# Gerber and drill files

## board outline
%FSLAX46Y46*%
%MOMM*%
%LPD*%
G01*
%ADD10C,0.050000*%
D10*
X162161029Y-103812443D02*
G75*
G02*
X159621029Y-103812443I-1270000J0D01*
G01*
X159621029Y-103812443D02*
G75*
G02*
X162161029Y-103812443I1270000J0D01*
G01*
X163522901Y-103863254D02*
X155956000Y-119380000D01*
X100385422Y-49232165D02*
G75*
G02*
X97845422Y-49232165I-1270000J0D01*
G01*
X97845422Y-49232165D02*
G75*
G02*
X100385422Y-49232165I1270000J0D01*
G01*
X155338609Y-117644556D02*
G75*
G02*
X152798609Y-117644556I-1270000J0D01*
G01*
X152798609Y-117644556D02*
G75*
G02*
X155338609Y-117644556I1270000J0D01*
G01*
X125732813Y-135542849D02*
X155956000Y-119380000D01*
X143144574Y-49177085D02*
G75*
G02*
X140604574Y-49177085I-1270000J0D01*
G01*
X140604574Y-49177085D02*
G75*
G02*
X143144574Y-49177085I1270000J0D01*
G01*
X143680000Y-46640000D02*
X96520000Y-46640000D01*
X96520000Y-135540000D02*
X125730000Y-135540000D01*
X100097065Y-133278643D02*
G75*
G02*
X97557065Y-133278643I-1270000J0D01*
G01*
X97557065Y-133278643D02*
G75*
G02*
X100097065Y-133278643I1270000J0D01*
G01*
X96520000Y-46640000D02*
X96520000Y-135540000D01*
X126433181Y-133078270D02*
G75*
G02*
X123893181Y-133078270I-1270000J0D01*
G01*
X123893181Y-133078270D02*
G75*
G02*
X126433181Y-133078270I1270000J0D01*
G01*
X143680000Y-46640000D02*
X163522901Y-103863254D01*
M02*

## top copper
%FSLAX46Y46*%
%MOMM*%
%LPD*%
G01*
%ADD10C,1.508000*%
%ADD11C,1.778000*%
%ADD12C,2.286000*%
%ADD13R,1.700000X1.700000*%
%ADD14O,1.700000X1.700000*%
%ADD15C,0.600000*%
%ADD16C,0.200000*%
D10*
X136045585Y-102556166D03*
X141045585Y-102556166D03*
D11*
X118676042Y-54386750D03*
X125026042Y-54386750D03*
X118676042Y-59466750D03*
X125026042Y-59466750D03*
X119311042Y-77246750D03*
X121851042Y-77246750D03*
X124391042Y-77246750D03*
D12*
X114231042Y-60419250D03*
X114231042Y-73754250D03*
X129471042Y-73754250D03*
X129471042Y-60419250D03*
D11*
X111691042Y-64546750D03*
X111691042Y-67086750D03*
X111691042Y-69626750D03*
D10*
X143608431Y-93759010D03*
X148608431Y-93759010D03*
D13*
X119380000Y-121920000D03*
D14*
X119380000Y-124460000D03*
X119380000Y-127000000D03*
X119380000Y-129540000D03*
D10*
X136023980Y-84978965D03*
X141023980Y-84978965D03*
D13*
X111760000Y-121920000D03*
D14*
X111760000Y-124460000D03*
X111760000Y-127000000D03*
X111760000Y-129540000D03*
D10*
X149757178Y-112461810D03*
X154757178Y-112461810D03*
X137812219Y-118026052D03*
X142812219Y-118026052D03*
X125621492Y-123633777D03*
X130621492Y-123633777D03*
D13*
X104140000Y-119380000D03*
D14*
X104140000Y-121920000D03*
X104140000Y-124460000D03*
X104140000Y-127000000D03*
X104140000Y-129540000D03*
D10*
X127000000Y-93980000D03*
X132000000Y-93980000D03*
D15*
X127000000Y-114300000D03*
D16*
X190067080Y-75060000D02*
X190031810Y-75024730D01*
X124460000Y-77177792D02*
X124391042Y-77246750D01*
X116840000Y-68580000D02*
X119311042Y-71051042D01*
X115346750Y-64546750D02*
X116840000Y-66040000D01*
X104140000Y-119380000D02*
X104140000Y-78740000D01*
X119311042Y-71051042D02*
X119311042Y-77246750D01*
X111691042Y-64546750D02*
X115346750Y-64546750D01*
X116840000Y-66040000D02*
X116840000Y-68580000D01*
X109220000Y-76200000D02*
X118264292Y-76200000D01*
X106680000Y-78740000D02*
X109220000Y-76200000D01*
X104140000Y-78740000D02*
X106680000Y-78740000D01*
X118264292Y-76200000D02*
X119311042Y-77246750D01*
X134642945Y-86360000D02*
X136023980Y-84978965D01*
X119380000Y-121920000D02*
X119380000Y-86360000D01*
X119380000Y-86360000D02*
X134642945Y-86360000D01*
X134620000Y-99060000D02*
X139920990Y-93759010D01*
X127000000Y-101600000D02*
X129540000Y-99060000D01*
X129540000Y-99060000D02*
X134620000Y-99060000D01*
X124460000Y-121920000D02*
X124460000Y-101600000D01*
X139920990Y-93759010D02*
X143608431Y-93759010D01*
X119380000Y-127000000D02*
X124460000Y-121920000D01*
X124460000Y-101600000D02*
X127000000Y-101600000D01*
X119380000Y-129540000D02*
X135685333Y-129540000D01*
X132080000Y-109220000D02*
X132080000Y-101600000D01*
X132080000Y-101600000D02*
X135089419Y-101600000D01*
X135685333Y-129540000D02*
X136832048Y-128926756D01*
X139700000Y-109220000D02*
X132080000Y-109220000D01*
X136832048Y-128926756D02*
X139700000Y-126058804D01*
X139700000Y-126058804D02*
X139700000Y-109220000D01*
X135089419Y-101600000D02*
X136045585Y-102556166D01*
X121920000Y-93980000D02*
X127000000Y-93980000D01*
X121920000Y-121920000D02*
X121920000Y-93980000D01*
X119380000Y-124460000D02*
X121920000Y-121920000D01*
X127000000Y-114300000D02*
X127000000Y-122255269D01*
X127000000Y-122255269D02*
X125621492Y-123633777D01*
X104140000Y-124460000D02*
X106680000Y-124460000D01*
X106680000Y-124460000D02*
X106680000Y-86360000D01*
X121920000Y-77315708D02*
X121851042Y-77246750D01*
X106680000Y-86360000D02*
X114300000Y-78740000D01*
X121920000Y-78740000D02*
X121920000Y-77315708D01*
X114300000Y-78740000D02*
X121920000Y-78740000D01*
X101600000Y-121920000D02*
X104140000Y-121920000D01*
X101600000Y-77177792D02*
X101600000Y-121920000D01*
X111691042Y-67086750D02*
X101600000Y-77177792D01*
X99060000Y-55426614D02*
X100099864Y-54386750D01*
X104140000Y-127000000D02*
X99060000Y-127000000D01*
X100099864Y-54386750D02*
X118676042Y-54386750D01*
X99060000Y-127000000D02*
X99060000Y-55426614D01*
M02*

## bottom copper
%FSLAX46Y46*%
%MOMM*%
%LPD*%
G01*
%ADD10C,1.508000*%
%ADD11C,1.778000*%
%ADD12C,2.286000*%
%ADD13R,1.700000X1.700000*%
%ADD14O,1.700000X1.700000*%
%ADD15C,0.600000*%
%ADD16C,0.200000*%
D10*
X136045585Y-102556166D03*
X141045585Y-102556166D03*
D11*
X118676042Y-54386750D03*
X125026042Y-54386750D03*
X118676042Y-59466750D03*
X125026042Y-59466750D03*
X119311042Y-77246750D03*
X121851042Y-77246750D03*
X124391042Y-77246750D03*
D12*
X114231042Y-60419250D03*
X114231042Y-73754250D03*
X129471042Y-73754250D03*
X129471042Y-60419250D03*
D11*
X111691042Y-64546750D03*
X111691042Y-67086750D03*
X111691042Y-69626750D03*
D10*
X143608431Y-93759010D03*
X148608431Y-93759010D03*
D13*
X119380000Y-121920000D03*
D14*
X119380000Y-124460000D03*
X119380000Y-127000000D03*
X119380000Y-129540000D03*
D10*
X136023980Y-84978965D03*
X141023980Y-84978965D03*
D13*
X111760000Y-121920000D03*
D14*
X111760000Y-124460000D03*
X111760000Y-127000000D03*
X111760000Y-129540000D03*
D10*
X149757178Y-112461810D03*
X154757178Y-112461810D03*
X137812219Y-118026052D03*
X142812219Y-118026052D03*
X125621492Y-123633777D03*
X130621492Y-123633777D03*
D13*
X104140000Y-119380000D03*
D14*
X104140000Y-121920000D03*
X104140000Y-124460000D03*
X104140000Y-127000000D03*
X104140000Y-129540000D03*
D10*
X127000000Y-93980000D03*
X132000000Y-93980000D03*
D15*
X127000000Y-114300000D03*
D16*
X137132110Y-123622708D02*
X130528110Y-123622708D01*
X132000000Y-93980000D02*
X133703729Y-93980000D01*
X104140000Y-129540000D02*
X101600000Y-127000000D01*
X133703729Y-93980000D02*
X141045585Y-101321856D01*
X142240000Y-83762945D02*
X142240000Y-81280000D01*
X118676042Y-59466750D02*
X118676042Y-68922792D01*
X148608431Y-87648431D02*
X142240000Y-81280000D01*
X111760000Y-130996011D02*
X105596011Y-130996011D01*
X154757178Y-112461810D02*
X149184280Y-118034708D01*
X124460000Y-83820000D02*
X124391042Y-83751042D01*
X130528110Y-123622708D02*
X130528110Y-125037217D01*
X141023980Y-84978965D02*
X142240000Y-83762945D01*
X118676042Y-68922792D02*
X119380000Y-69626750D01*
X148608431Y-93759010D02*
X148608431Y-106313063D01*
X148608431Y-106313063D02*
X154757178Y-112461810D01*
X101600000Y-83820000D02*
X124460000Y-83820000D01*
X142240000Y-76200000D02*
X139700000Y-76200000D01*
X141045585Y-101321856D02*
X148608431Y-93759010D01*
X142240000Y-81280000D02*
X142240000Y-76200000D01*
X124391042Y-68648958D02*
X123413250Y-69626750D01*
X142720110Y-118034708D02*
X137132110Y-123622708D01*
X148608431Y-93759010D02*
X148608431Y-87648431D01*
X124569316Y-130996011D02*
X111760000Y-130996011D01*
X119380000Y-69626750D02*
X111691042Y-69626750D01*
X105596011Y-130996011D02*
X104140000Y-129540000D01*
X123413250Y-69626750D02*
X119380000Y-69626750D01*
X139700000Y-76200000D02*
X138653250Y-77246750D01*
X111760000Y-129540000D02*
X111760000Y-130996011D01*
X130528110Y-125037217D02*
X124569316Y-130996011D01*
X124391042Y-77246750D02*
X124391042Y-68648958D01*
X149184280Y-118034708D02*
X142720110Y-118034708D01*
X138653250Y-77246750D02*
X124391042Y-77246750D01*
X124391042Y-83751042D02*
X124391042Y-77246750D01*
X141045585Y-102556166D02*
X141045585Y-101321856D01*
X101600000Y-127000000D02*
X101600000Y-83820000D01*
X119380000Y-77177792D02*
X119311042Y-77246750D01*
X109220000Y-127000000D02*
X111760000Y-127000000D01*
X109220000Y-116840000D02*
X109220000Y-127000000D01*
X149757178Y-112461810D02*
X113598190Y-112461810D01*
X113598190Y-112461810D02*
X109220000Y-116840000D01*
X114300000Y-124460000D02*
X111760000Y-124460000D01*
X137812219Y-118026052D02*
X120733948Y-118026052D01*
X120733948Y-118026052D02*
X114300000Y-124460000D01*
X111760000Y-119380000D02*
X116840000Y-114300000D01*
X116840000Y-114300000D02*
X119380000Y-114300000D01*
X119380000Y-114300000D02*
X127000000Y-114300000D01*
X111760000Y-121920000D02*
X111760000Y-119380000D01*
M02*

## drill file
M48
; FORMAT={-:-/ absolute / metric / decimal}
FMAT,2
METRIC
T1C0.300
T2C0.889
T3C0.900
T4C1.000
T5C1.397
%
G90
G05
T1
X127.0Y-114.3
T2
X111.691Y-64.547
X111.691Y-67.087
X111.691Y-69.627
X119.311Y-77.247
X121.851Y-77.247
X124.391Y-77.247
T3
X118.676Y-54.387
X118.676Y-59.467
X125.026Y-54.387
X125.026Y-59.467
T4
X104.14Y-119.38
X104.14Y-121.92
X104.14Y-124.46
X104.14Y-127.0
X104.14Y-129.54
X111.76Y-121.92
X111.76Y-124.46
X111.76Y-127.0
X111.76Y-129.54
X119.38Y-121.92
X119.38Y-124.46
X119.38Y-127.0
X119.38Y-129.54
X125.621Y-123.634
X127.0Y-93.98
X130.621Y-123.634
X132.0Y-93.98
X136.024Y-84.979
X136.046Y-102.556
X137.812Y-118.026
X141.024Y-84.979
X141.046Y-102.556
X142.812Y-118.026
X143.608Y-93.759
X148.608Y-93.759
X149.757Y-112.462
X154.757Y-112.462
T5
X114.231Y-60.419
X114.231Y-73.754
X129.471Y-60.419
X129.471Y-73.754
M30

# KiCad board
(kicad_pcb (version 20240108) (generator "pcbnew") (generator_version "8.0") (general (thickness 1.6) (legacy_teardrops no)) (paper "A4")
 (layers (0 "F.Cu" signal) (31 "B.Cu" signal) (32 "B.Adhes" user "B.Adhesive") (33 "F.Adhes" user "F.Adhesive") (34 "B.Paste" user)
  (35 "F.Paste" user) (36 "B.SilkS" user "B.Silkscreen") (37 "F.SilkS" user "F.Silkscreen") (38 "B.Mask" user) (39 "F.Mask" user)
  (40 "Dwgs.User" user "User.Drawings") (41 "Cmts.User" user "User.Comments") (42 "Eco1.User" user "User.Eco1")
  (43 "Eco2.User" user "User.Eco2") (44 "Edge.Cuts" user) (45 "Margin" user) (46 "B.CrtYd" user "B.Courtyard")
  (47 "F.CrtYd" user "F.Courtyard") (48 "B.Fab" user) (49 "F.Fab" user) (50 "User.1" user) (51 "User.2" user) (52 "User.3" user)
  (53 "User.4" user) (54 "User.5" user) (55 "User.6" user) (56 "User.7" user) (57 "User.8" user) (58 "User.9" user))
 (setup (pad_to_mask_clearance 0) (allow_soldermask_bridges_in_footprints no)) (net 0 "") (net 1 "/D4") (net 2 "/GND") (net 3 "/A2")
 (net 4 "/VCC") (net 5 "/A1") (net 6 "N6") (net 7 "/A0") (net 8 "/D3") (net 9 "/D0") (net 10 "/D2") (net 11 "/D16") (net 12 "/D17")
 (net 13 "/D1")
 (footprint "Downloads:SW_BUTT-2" (layer "F.Cu") (at 138.545585 102.556166)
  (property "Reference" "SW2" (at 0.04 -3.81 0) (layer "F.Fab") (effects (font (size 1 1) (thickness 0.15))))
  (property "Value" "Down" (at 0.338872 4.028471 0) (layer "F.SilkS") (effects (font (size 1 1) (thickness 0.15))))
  (pad "1" thru_hole circle (at -2.5 0) (size 1.508 1.508) (drill 1) (layers "*.Cu" "*.Mask") (remove_unused_layers no) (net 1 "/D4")
   (solder_mask_margin 0.102))
  (pad "2" thru_hole circle (at 2.5 0) (size 1.508 1.508) (drill 1) (layers "*.Cu" "*.Mask") (remove_unused_layers no) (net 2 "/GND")
   (solder_mask_margin 0.102)))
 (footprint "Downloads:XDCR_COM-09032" (layer "F.Cu") (at 121.851042 67.08675)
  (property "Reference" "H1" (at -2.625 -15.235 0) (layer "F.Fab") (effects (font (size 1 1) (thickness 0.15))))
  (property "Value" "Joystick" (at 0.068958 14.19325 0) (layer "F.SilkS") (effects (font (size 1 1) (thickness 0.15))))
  (pad "B1A" thru_hole circle (at -3.175 -12.7) (size 1.778 1.778) (drill 0.9) (layers "*.Cu" "*.Mask") (remove_unused_layers no)
   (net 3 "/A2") (solder_mask_margin 0.102))
  (pad "B1B" thru_hole circle (at 3.175 -12.7) (size 1.778 1.778) (drill 0.9) (layers "*.Cu" "*.Mask") (remove_unused_layers no)
   (solder_mask_margin 0.102))
  (pad "B2A" thru_hole circle (at -3.175 -7.62) (size 1.778 1.778) (drill 0.9) (layers "*.Cu" "*.Mask") (remove_unused_layers no)
   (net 2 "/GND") (solder_mask_margin 0.102))
  (pad "B2B" thru_hole circle (at 3.175 -7.62) (size 1.778 1.778) (drill 0.9) (layers "*.Cu" "*.Mask") (remove_unused_layers no)
   (solder_mask_margin 0.102))
  (pad "H1" thru_hole circle (at -2.54 10.16) (size 1.778 1.778) (drill 0.889) (layers "*.Cu" "*.Mask") (remove_unused_layers no)
   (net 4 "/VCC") (solder_mask_margin 0.102))
  (pad "H2" thru_hole circle (at 0 10.16) (size 1.778 1.778) (drill 0.889) (layers "*.Cu" "*.Mask") (remove_unused_layers no) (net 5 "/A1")
   (solder_mask_margin 0.102))
  (pad "H3" thru_hole circle (at 2.54 10.16) (size 1.778 1.778) (drill 0.889) (layers "*.Cu" "*.Mask") (remove_unused_layers no)
   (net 2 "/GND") (solder_mask_margin 0.102))
  (pad "S1" thru_hole circle (at -7.62 -6.6675) (size 2.286 2.286) (drill 1.397) (layers "*.Cu" "*.Mask") (remove_unused_layers no)
   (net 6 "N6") (solder_mask_margin 0.102))
  (pad "S2" thru_hole circle (at -7.62 6.6675) (size 2.286 2.286) (drill 1.397) (layers "*.Cu" "*.Mask") (remove_unused_layers no)
   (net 6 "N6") (solder_mask_margin 0.102))
  (pad "S3" thru_hole circle (at 7.62 6.6675) (size 2.286 2.286) (drill 1.397) (layers "*.Cu" "*.Mask") (remove_unused_layers no)
   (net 6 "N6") (solder_mask_margin 0.102))
  (pad "S4" thru_hole circle (at 7.62 -6.6675) (size 2.286 2.286) (drill 1.397) (layers "*.Cu" "*.Mask") (remove_unused_layers no)
   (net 6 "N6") (solder_mask_margin 0.102))
  (pad "V1" thru_hole circle (at -10.16 -2.54) (size 1.778 1.778) (drill 0.889) (layers "*.Cu" "*.Mask") (remove_unused_layers no)
   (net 4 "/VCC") (solder_mask_margin 0.102))
  (pad "V2" thru_hole circle (at -10.16 0) (size 1.778 1.778) (drill 0.889) (layers "*.Cu" "*.Mask") (remove_unused_layers no) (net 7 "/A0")
   (solder_mask_margin 0.102))
  (pad "V3" thru_hole circle (at -10.16 2.54) (size 1.778 1.778) (drill 0.889) (layers "*.Cu" "*.Mask") (remove_unused_layers no)
   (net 2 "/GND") (solder_mask_margin 0.102)))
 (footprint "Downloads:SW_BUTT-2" (layer "F.Cu") (at 146.108431 93.75901)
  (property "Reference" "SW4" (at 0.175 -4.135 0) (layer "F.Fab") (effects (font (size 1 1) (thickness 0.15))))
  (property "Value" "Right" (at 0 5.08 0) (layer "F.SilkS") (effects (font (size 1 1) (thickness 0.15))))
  (pad "1" thru_hole circle (at -2.5 0) (size 1.508 1.508) (drill 1) (layers "*.Cu" "*.Mask") (remove_unused_layers no) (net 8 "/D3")
   (solder_mask_margin 0.102))
  (pad "2" thru_hole circle (at 2.5 0) (size 1.508 1.508) (drill 1) (layers "*.Cu" "*.Mask") (remove_unused_layers no) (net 2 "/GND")
   (solder_mask_margin 0.102)))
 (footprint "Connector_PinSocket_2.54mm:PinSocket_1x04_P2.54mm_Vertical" (layer "F.Cu") (at 119.38 121.92)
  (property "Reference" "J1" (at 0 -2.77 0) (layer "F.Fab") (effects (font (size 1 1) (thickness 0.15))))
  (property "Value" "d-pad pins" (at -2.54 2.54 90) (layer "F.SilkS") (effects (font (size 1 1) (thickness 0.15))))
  (pad "1" thru_hole rect (at 0 0) (size 1.7 1.7) (drill 1) (layers "*.Cu" "*.Mask") (remove_unused_layers no) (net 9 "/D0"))
  (pad "2" thru_hole oval (at 0 2.54) (size 1.7 1.7) (drill 1) (layers "*.Cu" "*.Mask") (remove_unused_layers no) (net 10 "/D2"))
  (pad "3" thru_hole oval (at 0 5.08) (size 1.7 1.7) (drill 1) (layers "*.Cu" "*.Mask") (remove_unused_layers no) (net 8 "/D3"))
  (pad "4" thru_hole oval (at 0 7.62) (size 1.7 1.7) (drill 1) (layers "*.Cu" "*.Mask") (remove_unused_layers no) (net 1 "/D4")))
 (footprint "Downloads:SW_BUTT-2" (layer "F.Cu") (at 138.52398 84.978965)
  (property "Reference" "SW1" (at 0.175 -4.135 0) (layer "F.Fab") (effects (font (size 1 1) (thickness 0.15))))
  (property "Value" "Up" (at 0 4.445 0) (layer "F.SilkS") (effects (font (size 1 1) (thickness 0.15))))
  (pad "1" thru_hole circle (at -2.5 0) (size 1.508 1.508) (drill 1) (layers "*.Cu" "*.Mask") (remove_unused_layers no) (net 9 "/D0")
   (solder_mask_margin 0.102))
  (pad "2" thru_hole circle (at 2.5 0) (size 1.508 1.508) (drill 1) (layers "*.Cu" "*.Mask") (remove_unused_layers no) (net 2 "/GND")
   (solder_mask_margin 0.102)))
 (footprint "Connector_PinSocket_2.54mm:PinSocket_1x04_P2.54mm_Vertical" (layer "F.Cu") (at 111.76 121.92)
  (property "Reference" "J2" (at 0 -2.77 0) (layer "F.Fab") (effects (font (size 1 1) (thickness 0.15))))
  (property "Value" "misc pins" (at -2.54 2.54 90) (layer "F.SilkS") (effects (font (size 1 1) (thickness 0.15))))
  (pad "1" thru_hole rect (at 0 0) (size 1.7 1.7) (drill 1) (layers "*.Cu" "*.Mask") (remove_unused_layers no) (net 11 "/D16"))
  (pad "2" thru_hole oval (at 0 2.54) (size 1.7 1.7) (drill 1) (layers "*.Cu" "*.Mask") (remove_unused_layers no) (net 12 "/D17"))
  (pad "3" thru_hole oval (at 0 5.08) (size 1.7 1.7) (drill 1) (layers "*.Cu" "*.Mask") (remove_unused_layers no) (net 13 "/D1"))
  (pad "4" thru_hole oval (at 0 7.62) (size 1.7 1.7) (drill 1) (layers "*.Cu" "*.Mask") (remove_unused_layers no) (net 2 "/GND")))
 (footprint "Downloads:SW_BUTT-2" (layer "F.Cu") (at 152.257178 112.46181)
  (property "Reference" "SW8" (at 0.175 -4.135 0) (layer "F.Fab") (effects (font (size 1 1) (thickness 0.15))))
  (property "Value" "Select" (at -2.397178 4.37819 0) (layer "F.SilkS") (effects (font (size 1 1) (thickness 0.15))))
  (pad "1" thru_hole circle (at -2.5 0) (size 1.508 1.508) (drill 1) (layers "*.Cu" "*.Mask") (remove_unused_layers no) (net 13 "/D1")
   (solder_mask_margin 0.102))
  (pad "2" thru_hole circle (at 2.5 0) (size 1.508 1.508) (drill 1) (layers "*.Cu" "*.Mask") (remove_unused_layers no) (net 2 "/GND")
   (solder_mask_margin 0.102)))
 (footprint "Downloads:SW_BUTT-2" (layer "F.Cu") (at 140.312219 118.026052)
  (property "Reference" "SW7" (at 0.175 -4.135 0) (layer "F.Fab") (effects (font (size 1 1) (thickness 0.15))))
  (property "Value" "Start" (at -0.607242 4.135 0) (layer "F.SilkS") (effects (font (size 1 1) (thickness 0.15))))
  (pad "1" thru_hole circle (at -2.5 0) (size 1.508 1.508) (drill 1) (layers "*.Cu" "*.Mask") (remove_unused_layers no) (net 12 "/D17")
   (solder_mask_margin 0.102))
  (pad "2" thru_hole circle (at 2.5 0) (size 1.508 1.508) (drill 1) (layers "*.Cu" "*.Mask") (remove_unused_layers no) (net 2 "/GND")
   (solder_mask_margin 0.102)))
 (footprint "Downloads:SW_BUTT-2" (layer "F.Cu") (at 128.121492 123.633777)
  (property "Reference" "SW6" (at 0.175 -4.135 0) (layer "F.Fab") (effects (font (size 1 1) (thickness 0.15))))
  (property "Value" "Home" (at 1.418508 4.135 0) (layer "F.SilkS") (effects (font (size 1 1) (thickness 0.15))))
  (pad "1" thru_hole circle (at -2.5 0) (size 1.508 1.508) (drill 1) (layers "*.Cu" "*.Mask") (remove_unused_layers no) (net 11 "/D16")
   (solder_mask_margin 0.102))
  (pad "2" thru_hole circle (at 2.5 0) (size 1.508 1.508) (drill 1) (layers "*.Cu" "*.Mask") (remove_unused_layers no) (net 2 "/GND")
   (solder_mask_margin 0.102)))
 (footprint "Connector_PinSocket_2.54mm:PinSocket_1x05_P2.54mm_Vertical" (layer "F.Cu") (at 104.14 119.38)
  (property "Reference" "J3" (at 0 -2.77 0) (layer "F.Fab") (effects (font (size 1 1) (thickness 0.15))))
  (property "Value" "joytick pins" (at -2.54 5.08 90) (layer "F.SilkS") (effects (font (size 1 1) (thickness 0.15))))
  (pad "1" thru_hole rect (at 0 0) (size 1.7 1.7) (drill 1) (layers "*.Cu" "*.Mask") (remove_unused_layers no) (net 4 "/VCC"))
  (pad "2" thru_hole oval (at 0 2.54) (size 1.7 1.7) (drill 1) (layers "*.Cu" "*.Mask") (remove_unused_layers no) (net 7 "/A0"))
  (pad "3" thru_hole oval (at 0 5.08) (size 1.7 1.7) (drill 1) (layers "*.Cu" "*.Mask") (remove_unused_layers no) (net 5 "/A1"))
  (pad "4" thru_hole oval (at 0 7.62) (size 1.7 1.7) (drill 1) (layers "*.Cu" "*.Mask") (remove_unused_layers no) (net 3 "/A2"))
  (pad "5" thru_hole oval (at 0 10.16) (size 1.7 1.7) (drill 1) (layers "*.Cu" "*.Mask") (remove_unused_layers no) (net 2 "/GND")))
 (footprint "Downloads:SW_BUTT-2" (layer "F.Cu") (at 129.5 93.98)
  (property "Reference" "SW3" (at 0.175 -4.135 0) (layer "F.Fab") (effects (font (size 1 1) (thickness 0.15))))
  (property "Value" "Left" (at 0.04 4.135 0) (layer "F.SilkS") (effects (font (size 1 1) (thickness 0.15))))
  (pad "1" thru_hole circle (at -2.5 0) (size 1.508 1.508) (drill 1) (layers "*.Cu" "*.Mask") (remove_unused_layers no) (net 10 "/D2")
   (solder_mask_margin 0.102))
  (pad "2" thru_hole circle (at 2.5 0) (size 1.508 1.508) (drill 1) (layers "*.Cu" "*.Mask") (remove_unused_layers no) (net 2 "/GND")
   (solder_mask_margin 0.102)))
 (gr_circle (center 160.891029 103.812443) (end 162.161029 103.812443) (stroke (width 0.05) (type default)) (fill none) (layer "Edge.Cuts"))
 (gr_line (start 163.522901 103.863254) (end 155.956 119.38) (stroke (width 0.05) (type default)) (layer "Edge.Cuts"))
 (gr_circle (center 99.115422 49.232165) (end 97.845422 49.232165) (stroke (width 0.05) (type default)) (fill none) (layer "Edge.Cuts"))
 (gr_circle (center 154.068609 117.644556) (end 155.338609 117.644556) (stroke (width 0.05) (type default)) (fill none) (layer "Edge.Cuts"))
 (gr_line (start 125.732813 135.542849) (end 155.956 119.38) (stroke (width 0.05) (type default)) (layer "Edge.Cuts"))
 (gr_circle (center 141.874574 49.177085) (end 141.874574 47.907085) (stroke (width 0.05) (type default)) (fill none) (layer "Edge.Cuts"))
 (gr_line (start 143.68 46.64) (end 96.52 46.64) (stroke (width 0.05) (type default)) (layer "Edge.Cuts"))
 (gr_line (start 96.52 135.54) (end 125.73 135.54) (stroke (width 0.05) (type default)) (layer "Edge.Cuts"))
 (gr_circle (center 98.827065 133.278643) (end 100.097065 133.278643) (stroke (width 0.05) (type default)) (fill none) (layer "Edge.Cuts"))
 (gr_line (start 96.52 46.64) (end 96.52 135.54) (stroke (width 0.05) (type default)) (layer "Edge.Cuts"))
 (gr_circle (center 125.163181 133.07827) (end 126.433181 133.07827) (stroke (width 0.05) (type default)) (fill none) (layer "Edge.Cuts"))
 (gr_line (start 143.68 46.64) (end 163.522901 103.863254) (stroke (width 0.05) (type default)) (layer "Edge.Cuts"))
 (segment (start 190.06708 75.06) (end 190.03181 75.02473) (width 0.2) (layer "F.Cu") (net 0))
 (segment (start 124.46 77.177792) (end 124.391042 77.24675) (width 0.2) (layer "F.Cu") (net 2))
 (segment (start 137.13211 123.622708) (end 130.52811 123.622708) (width 0.2) (layer "B.Cu") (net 2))
 (segment (start 132 93.98) (end 133.703729 93.98) (width 0.2) (layer "B.Cu") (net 2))
 (segment (start 104.14 129.54) (end 101.6 127) (width 0.2) (layer "B.Cu") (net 2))
 (segment (start 133.703729 93.98) (end 141.045585 101.321856) (width 0.2) (layer "B.Cu") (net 2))
 (segment (start 142.24 83.762945) (end 142.24 81.28) (width 0.2) (layer "B.Cu") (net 2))
 (segment (start 118.676042 59.46675) (end 118.676042 68.922792) (width 0.2) (layer "B.Cu") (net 2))
 (segment (start 148.608431 87.648431) (end 142.24 81.28) (width 0.2) (layer "B.Cu") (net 2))
 (segment (start 111.76 130.996011) (end 105.596011 130.996011) (width 0.2) (layer "B.Cu") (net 2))
 (segment (start 154.757178 112.46181) (end 149.18428 118.034708) (width 0.2) (layer "B.Cu") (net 2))
 (segment (start 124.46 83.82) (end 124.391042 83.751042) (width 0.2) (layer "B.Cu") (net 2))
 (segment (start 130.52811 123.622708) (end 130.52811 125.037217) (width 0.2) (layer "B.Cu") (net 2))
 (segment (start 141.02398 84.978965) (end 142.24 83.762945) (width 0.2) (layer "B.Cu") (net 2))
 (segment (start 118.676042 68.922792) (end 119.38 69.62675) (width 0.2) (layer "B.Cu") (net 2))
 (segment (start 148.608431 93.75901) (end 148.608431 106.313063) (width 0.2) (layer "B.Cu") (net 2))
 (segment (start 148.608431 106.313063) (end 154.757178 112.46181) (width 0.2) (layer "B.Cu") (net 2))
 (segment (start 101.6 83.82) (end 124.46 83.82) (width 0.2) (layer "B.Cu") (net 2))
 (segment (start 142.24 76.2) (end 139.7 76.2) (width 0.2) (layer "B.Cu") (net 2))
 (segment (start 141.045585 101.321856) (end 148.608431 93.75901) (width 0.2) (layer "B.Cu") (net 2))
 (segment (start 142.24 81.28) (end 142.24 76.2) (width 0.2) (layer "B.Cu") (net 2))
 (segment (start 124.391042 68.648958) (end 123.41325 69.62675) (width 0.2) (layer "B.Cu") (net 2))
 (segment (start 142.72011 118.034708) (end 137.13211 123.622708) (width 0.2) (layer "B.Cu") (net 2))
 (segment (start 148.608431 93.75901) (end 148.608431 87.648431) (width 0.2) (layer "B.Cu") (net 2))
 (segment (start 124.569316 130.996011) (end 111.76 130.996011) (width 0.2) (layer "B.Cu") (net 2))
 (segment (start 119.38 69.62675) (end 111.691042 69.62675) (width 0.2) (layer "B.Cu") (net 2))
 (segment (start 105.596011 130.996011) (end 104.14 129.54) (width 0.2) (layer "B.Cu") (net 2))
 (segment (start 123.41325 69.62675) (end 119.38 69.62675) (width 0.2) (layer "B.Cu") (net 2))
 (segment (start 139.7 76.2) (end 138.65325 77.24675) (width 0.2) (layer "B.Cu") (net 2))
 (segment (start 111.76 129.54) (end 111.76 130.996011) (width 0.2) (layer "B.Cu") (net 2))
 (segment (start 130.52811 125.037217) (end 124.569316 130.996011) (width 0.2) (layer "B.Cu") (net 2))
 (segment (start 124.391042 77.24675) (end 124.391042 68.648958) (width 0.2) (layer "B.Cu") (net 2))
 (segment (start 149.18428 118.034708) (end 142.72011 118.034708) (width 0.2) (layer "B.Cu") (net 2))
 (segment (start 138.65325 77.24675) (end 124.391042 77.24675) (width 0.2) (layer "B.Cu") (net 2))
 (segment (start 124.391042 83.751042) (end 124.391042 77.24675) (width 0.2) (layer "B.Cu") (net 2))
 (segment (start 141.045585 102.556166) (end 141.045585 101.321856) (width 0.2) (layer "B.Cu") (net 2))
 (segment (start 101.6 127) (end 101.6 83.82) (width 0.2) (layer "B.Cu") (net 2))
 (segment (start 116.84 68.58) (end 119.311042 71.051042) (width 0.2) (layer "F.Cu") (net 4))
 (segment (start 115.34675 64.54675) (end 116.84 66.04) (width 0.2) (layer "F.Cu") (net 4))
 (segment (start 104.14 119.38) (end 104.14 78.74) (width 0.2) (layer "F.Cu") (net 4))
 (segment (start 119.311042 71.051042) (end 119.311042 77.24675) (width 0.2) (layer "F.Cu") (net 4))
 (segment (start 111.691042 64.54675) (end 115.34675 64.54675) (width 0.2) (layer "F.Cu") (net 4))
 (segment (start 116.84 66.04) (end 116.84 68.58) (width 0.2) (layer "F.Cu") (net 4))
 (segment (start 109.22 76.2) (end 118.264292 76.2) (width 0.2) (layer "F.Cu") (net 4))
 (segment (start 106.68 78.74) (end 109.22 76.2) (width 0.2) (layer "F.Cu") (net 4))
 (segment (start 104.14 78.74) (end 106.68 78.74) (width 0.2) (layer "F.Cu") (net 4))
 (segment (start 118.264292 76.2) (end 119.311042 77.24675) (width 0.2) (layer "F.Cu") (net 4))
 (segment (start 119.38 77.177792) (end 119.311042 77.24675) (width 0.2) (layer "B.Cu") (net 4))
 (segment (start 134.642945 86.36) (end 136.02398 84.978965) (width 0.2) (layer "F.Cu") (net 9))
 (segment (start 119.38 121.92) (end 119.38 86.36) (width 0.2) (layer "F.Cu") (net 9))
 (segment (start 119.38 86.36) (end 134.642945 86.36) (width 0.2) (layer "F.Cu") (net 9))
 (segment (start 134.62 99.06) (end 139.92099 93.75901) (width 0.2) (layer "F.Cu") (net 8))
 (segment (start 127 101.6) (end 129.54 99.06) (width 0.2) (layer "F.Cu") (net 8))
 (segment (start 129.54 99.06) (end 134.62 99.06) (width 0.2) (layer "F.Cu") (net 8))
 (segment (start 124.46 121.92) (end 124.46 101.6) (width 0.2) (layer "F.Cu") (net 8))
 (segment (start 139.92099 93.75901) (end 143.608431 93.75901) (width 0.2) (layer "F.Cu") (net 8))
 (segment (start 119.38 127) (end 124.46 121.92) (width 0.2) (layer "F.Cu") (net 8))
 (segment (start 124.46 101.6) (end 127 101.6) (width 0.2) (layer "F.Cu") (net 8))
 (segment (start 119.38 129.54) (end 135.685333 129.54) (width 0.2) (layer "F.Cu") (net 1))
 (segment (start 132.08 109.22) (end 132.08 101.6) (width 0.2) (layer "F.Cu") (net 1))
 (segment (start 132.08 101.6) (end 135.089419 101.6) (width 0.2) (layer "F.Cu") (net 1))
 (segment (start 135.685333 129.54) (end 136.832048 128.926756) (width 0.2) (layer "F.Cu") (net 1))
 (segment (start 139.7 109.22) (end 132.08 109.22) (width 0.2) (layer "F.Cu") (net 1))
 (segment (start 136.832048 128.926756) (end 139.7 126.058804) (width 0.2) (layer "F.Cu") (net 1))
 (segment (start 139.7 126.058804) (end 139.7 109.22) (width 0.2) (layer "F.Cu") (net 1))
 (segment (start 135.089419 101.6) (end 136.045585 102.556166) (width 0.2) (layer "F.Cu") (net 1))
 (segment (start 121.92 93.98) (end 127 93.98) (width 0.2) (layer "F.Cu") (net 10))
 (segment (start 121.92 121.92) (end 121.92 93.98) (width 0.2) (layer "F.Cu") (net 10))
 (segment (start 119.38 124.46) (end 121.92 121.92) (width 0.2) (layer "F.Cu") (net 10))
 (segment (start 109.22 127) (end 111.76 127) (width 0.2) (layer "B.Cu") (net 13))
 (segment (start 109.22 116.84) (end 109.22 127) (width 0.2) (layer "B.Cu") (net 13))
 (segment (start 149.757178 112.46181) (end 113.59819 112.46181) (width 0.2) (layer "B.Cu") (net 13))
 (segment (start 113.59819 112.46181) (end 109.22 116.84) (width 0.2) (layer "B.Cu") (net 13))
 (segment (start 114.3 124.46) (end 111.76 124.46) (width 0.2) (layer "B.Cu") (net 12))
 (segment (start 137.812219 118.026052) (end 120.733948 118.026052) (width 0.2) (layer "B.Cu") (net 12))
 (segment (start 120.733948 118.026052) (end 114.3 124.46) (width 0.2) (layer "B.Cu") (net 12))
 (segment (start 127 114.3) (end 127 122.255269) (width 0.2) (layer "F.Cu") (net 11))
 (segment (start 127 122.255269) (end 125.621492 123.633777) (width 0.2) (layer "F.Cu") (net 11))
 (via (at 127 114.3) (size 0.6) (drill 0.3) (layers "F.Cu" "B.Cu") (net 11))
 (segment (start 111.76 119.38) (end 116.84 114.3) (width 0.2) (layer "B.Cu") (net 11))
 (segment (start 116.84 114.3) (end 119.38 114.3) (width 0.2) (layer "B.Cu") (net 11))
 (segment (start 119.38 114.3) (end 127 114.3) (width 0.2) (layer "B.Cu") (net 11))
 (segment (start 111.76 121.92) (end 111.76 119.38) (width 0.2) (layer "B.Cu") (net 11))
 (segment (start 104.14 124.46) (end 106.68 124.46) (width 0.2) (layer "F.Cu") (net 5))
 (segment (start 106.68 124.46) (end 106.68 86.36) (width 0.2) (layer "F.Cu") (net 5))
 (segment (start 121.92 77.315708) (end 121.851042 77.24675) (width 0.2) (layer "F.Cu") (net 5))
 (segment (start 106.68 86.36) (end 114.3 78.74) (width 0.2) (layer "F.Cu") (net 5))
 (segment (start 121.92 78.74) (end 121.92 77.315708) (width 0.2) (layer "F.Cu") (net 5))
 (segment (start 114.3 78.74) (end 121.92 78.74) (width 0.2) (layer "F.Cu") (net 5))
 (segment (start 101.6 121.92) (end 104.14 121.92) (width 0.2) (layer "F.Cu") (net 7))
 (segment (start 101.6 77.177792) (end 101.6 121.92) (width 0.2) (layer "F.Cu") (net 7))
 (segment (start 111.691042 67.08675) (end 101.6 77.177792) (width 0.2) (layer "F.Cu") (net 7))
 (segment (start 99.06 55.426614) (end 100.099864 54.38675) (width 0.2) (layer "F.Cu") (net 3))
 (segment (start 104.14 127) (end 99.06 127) (width 0.2) (layer "F.Cu") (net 3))
 (segment (start 100.099864 54.38675) (end 118.676042 54.38675) (width 0.2) (layer "F.Cu") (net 3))
 (segment (start 99.06 127) (end 99.06 55.426614) (width 0.2) (layer "F.Cu") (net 3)))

